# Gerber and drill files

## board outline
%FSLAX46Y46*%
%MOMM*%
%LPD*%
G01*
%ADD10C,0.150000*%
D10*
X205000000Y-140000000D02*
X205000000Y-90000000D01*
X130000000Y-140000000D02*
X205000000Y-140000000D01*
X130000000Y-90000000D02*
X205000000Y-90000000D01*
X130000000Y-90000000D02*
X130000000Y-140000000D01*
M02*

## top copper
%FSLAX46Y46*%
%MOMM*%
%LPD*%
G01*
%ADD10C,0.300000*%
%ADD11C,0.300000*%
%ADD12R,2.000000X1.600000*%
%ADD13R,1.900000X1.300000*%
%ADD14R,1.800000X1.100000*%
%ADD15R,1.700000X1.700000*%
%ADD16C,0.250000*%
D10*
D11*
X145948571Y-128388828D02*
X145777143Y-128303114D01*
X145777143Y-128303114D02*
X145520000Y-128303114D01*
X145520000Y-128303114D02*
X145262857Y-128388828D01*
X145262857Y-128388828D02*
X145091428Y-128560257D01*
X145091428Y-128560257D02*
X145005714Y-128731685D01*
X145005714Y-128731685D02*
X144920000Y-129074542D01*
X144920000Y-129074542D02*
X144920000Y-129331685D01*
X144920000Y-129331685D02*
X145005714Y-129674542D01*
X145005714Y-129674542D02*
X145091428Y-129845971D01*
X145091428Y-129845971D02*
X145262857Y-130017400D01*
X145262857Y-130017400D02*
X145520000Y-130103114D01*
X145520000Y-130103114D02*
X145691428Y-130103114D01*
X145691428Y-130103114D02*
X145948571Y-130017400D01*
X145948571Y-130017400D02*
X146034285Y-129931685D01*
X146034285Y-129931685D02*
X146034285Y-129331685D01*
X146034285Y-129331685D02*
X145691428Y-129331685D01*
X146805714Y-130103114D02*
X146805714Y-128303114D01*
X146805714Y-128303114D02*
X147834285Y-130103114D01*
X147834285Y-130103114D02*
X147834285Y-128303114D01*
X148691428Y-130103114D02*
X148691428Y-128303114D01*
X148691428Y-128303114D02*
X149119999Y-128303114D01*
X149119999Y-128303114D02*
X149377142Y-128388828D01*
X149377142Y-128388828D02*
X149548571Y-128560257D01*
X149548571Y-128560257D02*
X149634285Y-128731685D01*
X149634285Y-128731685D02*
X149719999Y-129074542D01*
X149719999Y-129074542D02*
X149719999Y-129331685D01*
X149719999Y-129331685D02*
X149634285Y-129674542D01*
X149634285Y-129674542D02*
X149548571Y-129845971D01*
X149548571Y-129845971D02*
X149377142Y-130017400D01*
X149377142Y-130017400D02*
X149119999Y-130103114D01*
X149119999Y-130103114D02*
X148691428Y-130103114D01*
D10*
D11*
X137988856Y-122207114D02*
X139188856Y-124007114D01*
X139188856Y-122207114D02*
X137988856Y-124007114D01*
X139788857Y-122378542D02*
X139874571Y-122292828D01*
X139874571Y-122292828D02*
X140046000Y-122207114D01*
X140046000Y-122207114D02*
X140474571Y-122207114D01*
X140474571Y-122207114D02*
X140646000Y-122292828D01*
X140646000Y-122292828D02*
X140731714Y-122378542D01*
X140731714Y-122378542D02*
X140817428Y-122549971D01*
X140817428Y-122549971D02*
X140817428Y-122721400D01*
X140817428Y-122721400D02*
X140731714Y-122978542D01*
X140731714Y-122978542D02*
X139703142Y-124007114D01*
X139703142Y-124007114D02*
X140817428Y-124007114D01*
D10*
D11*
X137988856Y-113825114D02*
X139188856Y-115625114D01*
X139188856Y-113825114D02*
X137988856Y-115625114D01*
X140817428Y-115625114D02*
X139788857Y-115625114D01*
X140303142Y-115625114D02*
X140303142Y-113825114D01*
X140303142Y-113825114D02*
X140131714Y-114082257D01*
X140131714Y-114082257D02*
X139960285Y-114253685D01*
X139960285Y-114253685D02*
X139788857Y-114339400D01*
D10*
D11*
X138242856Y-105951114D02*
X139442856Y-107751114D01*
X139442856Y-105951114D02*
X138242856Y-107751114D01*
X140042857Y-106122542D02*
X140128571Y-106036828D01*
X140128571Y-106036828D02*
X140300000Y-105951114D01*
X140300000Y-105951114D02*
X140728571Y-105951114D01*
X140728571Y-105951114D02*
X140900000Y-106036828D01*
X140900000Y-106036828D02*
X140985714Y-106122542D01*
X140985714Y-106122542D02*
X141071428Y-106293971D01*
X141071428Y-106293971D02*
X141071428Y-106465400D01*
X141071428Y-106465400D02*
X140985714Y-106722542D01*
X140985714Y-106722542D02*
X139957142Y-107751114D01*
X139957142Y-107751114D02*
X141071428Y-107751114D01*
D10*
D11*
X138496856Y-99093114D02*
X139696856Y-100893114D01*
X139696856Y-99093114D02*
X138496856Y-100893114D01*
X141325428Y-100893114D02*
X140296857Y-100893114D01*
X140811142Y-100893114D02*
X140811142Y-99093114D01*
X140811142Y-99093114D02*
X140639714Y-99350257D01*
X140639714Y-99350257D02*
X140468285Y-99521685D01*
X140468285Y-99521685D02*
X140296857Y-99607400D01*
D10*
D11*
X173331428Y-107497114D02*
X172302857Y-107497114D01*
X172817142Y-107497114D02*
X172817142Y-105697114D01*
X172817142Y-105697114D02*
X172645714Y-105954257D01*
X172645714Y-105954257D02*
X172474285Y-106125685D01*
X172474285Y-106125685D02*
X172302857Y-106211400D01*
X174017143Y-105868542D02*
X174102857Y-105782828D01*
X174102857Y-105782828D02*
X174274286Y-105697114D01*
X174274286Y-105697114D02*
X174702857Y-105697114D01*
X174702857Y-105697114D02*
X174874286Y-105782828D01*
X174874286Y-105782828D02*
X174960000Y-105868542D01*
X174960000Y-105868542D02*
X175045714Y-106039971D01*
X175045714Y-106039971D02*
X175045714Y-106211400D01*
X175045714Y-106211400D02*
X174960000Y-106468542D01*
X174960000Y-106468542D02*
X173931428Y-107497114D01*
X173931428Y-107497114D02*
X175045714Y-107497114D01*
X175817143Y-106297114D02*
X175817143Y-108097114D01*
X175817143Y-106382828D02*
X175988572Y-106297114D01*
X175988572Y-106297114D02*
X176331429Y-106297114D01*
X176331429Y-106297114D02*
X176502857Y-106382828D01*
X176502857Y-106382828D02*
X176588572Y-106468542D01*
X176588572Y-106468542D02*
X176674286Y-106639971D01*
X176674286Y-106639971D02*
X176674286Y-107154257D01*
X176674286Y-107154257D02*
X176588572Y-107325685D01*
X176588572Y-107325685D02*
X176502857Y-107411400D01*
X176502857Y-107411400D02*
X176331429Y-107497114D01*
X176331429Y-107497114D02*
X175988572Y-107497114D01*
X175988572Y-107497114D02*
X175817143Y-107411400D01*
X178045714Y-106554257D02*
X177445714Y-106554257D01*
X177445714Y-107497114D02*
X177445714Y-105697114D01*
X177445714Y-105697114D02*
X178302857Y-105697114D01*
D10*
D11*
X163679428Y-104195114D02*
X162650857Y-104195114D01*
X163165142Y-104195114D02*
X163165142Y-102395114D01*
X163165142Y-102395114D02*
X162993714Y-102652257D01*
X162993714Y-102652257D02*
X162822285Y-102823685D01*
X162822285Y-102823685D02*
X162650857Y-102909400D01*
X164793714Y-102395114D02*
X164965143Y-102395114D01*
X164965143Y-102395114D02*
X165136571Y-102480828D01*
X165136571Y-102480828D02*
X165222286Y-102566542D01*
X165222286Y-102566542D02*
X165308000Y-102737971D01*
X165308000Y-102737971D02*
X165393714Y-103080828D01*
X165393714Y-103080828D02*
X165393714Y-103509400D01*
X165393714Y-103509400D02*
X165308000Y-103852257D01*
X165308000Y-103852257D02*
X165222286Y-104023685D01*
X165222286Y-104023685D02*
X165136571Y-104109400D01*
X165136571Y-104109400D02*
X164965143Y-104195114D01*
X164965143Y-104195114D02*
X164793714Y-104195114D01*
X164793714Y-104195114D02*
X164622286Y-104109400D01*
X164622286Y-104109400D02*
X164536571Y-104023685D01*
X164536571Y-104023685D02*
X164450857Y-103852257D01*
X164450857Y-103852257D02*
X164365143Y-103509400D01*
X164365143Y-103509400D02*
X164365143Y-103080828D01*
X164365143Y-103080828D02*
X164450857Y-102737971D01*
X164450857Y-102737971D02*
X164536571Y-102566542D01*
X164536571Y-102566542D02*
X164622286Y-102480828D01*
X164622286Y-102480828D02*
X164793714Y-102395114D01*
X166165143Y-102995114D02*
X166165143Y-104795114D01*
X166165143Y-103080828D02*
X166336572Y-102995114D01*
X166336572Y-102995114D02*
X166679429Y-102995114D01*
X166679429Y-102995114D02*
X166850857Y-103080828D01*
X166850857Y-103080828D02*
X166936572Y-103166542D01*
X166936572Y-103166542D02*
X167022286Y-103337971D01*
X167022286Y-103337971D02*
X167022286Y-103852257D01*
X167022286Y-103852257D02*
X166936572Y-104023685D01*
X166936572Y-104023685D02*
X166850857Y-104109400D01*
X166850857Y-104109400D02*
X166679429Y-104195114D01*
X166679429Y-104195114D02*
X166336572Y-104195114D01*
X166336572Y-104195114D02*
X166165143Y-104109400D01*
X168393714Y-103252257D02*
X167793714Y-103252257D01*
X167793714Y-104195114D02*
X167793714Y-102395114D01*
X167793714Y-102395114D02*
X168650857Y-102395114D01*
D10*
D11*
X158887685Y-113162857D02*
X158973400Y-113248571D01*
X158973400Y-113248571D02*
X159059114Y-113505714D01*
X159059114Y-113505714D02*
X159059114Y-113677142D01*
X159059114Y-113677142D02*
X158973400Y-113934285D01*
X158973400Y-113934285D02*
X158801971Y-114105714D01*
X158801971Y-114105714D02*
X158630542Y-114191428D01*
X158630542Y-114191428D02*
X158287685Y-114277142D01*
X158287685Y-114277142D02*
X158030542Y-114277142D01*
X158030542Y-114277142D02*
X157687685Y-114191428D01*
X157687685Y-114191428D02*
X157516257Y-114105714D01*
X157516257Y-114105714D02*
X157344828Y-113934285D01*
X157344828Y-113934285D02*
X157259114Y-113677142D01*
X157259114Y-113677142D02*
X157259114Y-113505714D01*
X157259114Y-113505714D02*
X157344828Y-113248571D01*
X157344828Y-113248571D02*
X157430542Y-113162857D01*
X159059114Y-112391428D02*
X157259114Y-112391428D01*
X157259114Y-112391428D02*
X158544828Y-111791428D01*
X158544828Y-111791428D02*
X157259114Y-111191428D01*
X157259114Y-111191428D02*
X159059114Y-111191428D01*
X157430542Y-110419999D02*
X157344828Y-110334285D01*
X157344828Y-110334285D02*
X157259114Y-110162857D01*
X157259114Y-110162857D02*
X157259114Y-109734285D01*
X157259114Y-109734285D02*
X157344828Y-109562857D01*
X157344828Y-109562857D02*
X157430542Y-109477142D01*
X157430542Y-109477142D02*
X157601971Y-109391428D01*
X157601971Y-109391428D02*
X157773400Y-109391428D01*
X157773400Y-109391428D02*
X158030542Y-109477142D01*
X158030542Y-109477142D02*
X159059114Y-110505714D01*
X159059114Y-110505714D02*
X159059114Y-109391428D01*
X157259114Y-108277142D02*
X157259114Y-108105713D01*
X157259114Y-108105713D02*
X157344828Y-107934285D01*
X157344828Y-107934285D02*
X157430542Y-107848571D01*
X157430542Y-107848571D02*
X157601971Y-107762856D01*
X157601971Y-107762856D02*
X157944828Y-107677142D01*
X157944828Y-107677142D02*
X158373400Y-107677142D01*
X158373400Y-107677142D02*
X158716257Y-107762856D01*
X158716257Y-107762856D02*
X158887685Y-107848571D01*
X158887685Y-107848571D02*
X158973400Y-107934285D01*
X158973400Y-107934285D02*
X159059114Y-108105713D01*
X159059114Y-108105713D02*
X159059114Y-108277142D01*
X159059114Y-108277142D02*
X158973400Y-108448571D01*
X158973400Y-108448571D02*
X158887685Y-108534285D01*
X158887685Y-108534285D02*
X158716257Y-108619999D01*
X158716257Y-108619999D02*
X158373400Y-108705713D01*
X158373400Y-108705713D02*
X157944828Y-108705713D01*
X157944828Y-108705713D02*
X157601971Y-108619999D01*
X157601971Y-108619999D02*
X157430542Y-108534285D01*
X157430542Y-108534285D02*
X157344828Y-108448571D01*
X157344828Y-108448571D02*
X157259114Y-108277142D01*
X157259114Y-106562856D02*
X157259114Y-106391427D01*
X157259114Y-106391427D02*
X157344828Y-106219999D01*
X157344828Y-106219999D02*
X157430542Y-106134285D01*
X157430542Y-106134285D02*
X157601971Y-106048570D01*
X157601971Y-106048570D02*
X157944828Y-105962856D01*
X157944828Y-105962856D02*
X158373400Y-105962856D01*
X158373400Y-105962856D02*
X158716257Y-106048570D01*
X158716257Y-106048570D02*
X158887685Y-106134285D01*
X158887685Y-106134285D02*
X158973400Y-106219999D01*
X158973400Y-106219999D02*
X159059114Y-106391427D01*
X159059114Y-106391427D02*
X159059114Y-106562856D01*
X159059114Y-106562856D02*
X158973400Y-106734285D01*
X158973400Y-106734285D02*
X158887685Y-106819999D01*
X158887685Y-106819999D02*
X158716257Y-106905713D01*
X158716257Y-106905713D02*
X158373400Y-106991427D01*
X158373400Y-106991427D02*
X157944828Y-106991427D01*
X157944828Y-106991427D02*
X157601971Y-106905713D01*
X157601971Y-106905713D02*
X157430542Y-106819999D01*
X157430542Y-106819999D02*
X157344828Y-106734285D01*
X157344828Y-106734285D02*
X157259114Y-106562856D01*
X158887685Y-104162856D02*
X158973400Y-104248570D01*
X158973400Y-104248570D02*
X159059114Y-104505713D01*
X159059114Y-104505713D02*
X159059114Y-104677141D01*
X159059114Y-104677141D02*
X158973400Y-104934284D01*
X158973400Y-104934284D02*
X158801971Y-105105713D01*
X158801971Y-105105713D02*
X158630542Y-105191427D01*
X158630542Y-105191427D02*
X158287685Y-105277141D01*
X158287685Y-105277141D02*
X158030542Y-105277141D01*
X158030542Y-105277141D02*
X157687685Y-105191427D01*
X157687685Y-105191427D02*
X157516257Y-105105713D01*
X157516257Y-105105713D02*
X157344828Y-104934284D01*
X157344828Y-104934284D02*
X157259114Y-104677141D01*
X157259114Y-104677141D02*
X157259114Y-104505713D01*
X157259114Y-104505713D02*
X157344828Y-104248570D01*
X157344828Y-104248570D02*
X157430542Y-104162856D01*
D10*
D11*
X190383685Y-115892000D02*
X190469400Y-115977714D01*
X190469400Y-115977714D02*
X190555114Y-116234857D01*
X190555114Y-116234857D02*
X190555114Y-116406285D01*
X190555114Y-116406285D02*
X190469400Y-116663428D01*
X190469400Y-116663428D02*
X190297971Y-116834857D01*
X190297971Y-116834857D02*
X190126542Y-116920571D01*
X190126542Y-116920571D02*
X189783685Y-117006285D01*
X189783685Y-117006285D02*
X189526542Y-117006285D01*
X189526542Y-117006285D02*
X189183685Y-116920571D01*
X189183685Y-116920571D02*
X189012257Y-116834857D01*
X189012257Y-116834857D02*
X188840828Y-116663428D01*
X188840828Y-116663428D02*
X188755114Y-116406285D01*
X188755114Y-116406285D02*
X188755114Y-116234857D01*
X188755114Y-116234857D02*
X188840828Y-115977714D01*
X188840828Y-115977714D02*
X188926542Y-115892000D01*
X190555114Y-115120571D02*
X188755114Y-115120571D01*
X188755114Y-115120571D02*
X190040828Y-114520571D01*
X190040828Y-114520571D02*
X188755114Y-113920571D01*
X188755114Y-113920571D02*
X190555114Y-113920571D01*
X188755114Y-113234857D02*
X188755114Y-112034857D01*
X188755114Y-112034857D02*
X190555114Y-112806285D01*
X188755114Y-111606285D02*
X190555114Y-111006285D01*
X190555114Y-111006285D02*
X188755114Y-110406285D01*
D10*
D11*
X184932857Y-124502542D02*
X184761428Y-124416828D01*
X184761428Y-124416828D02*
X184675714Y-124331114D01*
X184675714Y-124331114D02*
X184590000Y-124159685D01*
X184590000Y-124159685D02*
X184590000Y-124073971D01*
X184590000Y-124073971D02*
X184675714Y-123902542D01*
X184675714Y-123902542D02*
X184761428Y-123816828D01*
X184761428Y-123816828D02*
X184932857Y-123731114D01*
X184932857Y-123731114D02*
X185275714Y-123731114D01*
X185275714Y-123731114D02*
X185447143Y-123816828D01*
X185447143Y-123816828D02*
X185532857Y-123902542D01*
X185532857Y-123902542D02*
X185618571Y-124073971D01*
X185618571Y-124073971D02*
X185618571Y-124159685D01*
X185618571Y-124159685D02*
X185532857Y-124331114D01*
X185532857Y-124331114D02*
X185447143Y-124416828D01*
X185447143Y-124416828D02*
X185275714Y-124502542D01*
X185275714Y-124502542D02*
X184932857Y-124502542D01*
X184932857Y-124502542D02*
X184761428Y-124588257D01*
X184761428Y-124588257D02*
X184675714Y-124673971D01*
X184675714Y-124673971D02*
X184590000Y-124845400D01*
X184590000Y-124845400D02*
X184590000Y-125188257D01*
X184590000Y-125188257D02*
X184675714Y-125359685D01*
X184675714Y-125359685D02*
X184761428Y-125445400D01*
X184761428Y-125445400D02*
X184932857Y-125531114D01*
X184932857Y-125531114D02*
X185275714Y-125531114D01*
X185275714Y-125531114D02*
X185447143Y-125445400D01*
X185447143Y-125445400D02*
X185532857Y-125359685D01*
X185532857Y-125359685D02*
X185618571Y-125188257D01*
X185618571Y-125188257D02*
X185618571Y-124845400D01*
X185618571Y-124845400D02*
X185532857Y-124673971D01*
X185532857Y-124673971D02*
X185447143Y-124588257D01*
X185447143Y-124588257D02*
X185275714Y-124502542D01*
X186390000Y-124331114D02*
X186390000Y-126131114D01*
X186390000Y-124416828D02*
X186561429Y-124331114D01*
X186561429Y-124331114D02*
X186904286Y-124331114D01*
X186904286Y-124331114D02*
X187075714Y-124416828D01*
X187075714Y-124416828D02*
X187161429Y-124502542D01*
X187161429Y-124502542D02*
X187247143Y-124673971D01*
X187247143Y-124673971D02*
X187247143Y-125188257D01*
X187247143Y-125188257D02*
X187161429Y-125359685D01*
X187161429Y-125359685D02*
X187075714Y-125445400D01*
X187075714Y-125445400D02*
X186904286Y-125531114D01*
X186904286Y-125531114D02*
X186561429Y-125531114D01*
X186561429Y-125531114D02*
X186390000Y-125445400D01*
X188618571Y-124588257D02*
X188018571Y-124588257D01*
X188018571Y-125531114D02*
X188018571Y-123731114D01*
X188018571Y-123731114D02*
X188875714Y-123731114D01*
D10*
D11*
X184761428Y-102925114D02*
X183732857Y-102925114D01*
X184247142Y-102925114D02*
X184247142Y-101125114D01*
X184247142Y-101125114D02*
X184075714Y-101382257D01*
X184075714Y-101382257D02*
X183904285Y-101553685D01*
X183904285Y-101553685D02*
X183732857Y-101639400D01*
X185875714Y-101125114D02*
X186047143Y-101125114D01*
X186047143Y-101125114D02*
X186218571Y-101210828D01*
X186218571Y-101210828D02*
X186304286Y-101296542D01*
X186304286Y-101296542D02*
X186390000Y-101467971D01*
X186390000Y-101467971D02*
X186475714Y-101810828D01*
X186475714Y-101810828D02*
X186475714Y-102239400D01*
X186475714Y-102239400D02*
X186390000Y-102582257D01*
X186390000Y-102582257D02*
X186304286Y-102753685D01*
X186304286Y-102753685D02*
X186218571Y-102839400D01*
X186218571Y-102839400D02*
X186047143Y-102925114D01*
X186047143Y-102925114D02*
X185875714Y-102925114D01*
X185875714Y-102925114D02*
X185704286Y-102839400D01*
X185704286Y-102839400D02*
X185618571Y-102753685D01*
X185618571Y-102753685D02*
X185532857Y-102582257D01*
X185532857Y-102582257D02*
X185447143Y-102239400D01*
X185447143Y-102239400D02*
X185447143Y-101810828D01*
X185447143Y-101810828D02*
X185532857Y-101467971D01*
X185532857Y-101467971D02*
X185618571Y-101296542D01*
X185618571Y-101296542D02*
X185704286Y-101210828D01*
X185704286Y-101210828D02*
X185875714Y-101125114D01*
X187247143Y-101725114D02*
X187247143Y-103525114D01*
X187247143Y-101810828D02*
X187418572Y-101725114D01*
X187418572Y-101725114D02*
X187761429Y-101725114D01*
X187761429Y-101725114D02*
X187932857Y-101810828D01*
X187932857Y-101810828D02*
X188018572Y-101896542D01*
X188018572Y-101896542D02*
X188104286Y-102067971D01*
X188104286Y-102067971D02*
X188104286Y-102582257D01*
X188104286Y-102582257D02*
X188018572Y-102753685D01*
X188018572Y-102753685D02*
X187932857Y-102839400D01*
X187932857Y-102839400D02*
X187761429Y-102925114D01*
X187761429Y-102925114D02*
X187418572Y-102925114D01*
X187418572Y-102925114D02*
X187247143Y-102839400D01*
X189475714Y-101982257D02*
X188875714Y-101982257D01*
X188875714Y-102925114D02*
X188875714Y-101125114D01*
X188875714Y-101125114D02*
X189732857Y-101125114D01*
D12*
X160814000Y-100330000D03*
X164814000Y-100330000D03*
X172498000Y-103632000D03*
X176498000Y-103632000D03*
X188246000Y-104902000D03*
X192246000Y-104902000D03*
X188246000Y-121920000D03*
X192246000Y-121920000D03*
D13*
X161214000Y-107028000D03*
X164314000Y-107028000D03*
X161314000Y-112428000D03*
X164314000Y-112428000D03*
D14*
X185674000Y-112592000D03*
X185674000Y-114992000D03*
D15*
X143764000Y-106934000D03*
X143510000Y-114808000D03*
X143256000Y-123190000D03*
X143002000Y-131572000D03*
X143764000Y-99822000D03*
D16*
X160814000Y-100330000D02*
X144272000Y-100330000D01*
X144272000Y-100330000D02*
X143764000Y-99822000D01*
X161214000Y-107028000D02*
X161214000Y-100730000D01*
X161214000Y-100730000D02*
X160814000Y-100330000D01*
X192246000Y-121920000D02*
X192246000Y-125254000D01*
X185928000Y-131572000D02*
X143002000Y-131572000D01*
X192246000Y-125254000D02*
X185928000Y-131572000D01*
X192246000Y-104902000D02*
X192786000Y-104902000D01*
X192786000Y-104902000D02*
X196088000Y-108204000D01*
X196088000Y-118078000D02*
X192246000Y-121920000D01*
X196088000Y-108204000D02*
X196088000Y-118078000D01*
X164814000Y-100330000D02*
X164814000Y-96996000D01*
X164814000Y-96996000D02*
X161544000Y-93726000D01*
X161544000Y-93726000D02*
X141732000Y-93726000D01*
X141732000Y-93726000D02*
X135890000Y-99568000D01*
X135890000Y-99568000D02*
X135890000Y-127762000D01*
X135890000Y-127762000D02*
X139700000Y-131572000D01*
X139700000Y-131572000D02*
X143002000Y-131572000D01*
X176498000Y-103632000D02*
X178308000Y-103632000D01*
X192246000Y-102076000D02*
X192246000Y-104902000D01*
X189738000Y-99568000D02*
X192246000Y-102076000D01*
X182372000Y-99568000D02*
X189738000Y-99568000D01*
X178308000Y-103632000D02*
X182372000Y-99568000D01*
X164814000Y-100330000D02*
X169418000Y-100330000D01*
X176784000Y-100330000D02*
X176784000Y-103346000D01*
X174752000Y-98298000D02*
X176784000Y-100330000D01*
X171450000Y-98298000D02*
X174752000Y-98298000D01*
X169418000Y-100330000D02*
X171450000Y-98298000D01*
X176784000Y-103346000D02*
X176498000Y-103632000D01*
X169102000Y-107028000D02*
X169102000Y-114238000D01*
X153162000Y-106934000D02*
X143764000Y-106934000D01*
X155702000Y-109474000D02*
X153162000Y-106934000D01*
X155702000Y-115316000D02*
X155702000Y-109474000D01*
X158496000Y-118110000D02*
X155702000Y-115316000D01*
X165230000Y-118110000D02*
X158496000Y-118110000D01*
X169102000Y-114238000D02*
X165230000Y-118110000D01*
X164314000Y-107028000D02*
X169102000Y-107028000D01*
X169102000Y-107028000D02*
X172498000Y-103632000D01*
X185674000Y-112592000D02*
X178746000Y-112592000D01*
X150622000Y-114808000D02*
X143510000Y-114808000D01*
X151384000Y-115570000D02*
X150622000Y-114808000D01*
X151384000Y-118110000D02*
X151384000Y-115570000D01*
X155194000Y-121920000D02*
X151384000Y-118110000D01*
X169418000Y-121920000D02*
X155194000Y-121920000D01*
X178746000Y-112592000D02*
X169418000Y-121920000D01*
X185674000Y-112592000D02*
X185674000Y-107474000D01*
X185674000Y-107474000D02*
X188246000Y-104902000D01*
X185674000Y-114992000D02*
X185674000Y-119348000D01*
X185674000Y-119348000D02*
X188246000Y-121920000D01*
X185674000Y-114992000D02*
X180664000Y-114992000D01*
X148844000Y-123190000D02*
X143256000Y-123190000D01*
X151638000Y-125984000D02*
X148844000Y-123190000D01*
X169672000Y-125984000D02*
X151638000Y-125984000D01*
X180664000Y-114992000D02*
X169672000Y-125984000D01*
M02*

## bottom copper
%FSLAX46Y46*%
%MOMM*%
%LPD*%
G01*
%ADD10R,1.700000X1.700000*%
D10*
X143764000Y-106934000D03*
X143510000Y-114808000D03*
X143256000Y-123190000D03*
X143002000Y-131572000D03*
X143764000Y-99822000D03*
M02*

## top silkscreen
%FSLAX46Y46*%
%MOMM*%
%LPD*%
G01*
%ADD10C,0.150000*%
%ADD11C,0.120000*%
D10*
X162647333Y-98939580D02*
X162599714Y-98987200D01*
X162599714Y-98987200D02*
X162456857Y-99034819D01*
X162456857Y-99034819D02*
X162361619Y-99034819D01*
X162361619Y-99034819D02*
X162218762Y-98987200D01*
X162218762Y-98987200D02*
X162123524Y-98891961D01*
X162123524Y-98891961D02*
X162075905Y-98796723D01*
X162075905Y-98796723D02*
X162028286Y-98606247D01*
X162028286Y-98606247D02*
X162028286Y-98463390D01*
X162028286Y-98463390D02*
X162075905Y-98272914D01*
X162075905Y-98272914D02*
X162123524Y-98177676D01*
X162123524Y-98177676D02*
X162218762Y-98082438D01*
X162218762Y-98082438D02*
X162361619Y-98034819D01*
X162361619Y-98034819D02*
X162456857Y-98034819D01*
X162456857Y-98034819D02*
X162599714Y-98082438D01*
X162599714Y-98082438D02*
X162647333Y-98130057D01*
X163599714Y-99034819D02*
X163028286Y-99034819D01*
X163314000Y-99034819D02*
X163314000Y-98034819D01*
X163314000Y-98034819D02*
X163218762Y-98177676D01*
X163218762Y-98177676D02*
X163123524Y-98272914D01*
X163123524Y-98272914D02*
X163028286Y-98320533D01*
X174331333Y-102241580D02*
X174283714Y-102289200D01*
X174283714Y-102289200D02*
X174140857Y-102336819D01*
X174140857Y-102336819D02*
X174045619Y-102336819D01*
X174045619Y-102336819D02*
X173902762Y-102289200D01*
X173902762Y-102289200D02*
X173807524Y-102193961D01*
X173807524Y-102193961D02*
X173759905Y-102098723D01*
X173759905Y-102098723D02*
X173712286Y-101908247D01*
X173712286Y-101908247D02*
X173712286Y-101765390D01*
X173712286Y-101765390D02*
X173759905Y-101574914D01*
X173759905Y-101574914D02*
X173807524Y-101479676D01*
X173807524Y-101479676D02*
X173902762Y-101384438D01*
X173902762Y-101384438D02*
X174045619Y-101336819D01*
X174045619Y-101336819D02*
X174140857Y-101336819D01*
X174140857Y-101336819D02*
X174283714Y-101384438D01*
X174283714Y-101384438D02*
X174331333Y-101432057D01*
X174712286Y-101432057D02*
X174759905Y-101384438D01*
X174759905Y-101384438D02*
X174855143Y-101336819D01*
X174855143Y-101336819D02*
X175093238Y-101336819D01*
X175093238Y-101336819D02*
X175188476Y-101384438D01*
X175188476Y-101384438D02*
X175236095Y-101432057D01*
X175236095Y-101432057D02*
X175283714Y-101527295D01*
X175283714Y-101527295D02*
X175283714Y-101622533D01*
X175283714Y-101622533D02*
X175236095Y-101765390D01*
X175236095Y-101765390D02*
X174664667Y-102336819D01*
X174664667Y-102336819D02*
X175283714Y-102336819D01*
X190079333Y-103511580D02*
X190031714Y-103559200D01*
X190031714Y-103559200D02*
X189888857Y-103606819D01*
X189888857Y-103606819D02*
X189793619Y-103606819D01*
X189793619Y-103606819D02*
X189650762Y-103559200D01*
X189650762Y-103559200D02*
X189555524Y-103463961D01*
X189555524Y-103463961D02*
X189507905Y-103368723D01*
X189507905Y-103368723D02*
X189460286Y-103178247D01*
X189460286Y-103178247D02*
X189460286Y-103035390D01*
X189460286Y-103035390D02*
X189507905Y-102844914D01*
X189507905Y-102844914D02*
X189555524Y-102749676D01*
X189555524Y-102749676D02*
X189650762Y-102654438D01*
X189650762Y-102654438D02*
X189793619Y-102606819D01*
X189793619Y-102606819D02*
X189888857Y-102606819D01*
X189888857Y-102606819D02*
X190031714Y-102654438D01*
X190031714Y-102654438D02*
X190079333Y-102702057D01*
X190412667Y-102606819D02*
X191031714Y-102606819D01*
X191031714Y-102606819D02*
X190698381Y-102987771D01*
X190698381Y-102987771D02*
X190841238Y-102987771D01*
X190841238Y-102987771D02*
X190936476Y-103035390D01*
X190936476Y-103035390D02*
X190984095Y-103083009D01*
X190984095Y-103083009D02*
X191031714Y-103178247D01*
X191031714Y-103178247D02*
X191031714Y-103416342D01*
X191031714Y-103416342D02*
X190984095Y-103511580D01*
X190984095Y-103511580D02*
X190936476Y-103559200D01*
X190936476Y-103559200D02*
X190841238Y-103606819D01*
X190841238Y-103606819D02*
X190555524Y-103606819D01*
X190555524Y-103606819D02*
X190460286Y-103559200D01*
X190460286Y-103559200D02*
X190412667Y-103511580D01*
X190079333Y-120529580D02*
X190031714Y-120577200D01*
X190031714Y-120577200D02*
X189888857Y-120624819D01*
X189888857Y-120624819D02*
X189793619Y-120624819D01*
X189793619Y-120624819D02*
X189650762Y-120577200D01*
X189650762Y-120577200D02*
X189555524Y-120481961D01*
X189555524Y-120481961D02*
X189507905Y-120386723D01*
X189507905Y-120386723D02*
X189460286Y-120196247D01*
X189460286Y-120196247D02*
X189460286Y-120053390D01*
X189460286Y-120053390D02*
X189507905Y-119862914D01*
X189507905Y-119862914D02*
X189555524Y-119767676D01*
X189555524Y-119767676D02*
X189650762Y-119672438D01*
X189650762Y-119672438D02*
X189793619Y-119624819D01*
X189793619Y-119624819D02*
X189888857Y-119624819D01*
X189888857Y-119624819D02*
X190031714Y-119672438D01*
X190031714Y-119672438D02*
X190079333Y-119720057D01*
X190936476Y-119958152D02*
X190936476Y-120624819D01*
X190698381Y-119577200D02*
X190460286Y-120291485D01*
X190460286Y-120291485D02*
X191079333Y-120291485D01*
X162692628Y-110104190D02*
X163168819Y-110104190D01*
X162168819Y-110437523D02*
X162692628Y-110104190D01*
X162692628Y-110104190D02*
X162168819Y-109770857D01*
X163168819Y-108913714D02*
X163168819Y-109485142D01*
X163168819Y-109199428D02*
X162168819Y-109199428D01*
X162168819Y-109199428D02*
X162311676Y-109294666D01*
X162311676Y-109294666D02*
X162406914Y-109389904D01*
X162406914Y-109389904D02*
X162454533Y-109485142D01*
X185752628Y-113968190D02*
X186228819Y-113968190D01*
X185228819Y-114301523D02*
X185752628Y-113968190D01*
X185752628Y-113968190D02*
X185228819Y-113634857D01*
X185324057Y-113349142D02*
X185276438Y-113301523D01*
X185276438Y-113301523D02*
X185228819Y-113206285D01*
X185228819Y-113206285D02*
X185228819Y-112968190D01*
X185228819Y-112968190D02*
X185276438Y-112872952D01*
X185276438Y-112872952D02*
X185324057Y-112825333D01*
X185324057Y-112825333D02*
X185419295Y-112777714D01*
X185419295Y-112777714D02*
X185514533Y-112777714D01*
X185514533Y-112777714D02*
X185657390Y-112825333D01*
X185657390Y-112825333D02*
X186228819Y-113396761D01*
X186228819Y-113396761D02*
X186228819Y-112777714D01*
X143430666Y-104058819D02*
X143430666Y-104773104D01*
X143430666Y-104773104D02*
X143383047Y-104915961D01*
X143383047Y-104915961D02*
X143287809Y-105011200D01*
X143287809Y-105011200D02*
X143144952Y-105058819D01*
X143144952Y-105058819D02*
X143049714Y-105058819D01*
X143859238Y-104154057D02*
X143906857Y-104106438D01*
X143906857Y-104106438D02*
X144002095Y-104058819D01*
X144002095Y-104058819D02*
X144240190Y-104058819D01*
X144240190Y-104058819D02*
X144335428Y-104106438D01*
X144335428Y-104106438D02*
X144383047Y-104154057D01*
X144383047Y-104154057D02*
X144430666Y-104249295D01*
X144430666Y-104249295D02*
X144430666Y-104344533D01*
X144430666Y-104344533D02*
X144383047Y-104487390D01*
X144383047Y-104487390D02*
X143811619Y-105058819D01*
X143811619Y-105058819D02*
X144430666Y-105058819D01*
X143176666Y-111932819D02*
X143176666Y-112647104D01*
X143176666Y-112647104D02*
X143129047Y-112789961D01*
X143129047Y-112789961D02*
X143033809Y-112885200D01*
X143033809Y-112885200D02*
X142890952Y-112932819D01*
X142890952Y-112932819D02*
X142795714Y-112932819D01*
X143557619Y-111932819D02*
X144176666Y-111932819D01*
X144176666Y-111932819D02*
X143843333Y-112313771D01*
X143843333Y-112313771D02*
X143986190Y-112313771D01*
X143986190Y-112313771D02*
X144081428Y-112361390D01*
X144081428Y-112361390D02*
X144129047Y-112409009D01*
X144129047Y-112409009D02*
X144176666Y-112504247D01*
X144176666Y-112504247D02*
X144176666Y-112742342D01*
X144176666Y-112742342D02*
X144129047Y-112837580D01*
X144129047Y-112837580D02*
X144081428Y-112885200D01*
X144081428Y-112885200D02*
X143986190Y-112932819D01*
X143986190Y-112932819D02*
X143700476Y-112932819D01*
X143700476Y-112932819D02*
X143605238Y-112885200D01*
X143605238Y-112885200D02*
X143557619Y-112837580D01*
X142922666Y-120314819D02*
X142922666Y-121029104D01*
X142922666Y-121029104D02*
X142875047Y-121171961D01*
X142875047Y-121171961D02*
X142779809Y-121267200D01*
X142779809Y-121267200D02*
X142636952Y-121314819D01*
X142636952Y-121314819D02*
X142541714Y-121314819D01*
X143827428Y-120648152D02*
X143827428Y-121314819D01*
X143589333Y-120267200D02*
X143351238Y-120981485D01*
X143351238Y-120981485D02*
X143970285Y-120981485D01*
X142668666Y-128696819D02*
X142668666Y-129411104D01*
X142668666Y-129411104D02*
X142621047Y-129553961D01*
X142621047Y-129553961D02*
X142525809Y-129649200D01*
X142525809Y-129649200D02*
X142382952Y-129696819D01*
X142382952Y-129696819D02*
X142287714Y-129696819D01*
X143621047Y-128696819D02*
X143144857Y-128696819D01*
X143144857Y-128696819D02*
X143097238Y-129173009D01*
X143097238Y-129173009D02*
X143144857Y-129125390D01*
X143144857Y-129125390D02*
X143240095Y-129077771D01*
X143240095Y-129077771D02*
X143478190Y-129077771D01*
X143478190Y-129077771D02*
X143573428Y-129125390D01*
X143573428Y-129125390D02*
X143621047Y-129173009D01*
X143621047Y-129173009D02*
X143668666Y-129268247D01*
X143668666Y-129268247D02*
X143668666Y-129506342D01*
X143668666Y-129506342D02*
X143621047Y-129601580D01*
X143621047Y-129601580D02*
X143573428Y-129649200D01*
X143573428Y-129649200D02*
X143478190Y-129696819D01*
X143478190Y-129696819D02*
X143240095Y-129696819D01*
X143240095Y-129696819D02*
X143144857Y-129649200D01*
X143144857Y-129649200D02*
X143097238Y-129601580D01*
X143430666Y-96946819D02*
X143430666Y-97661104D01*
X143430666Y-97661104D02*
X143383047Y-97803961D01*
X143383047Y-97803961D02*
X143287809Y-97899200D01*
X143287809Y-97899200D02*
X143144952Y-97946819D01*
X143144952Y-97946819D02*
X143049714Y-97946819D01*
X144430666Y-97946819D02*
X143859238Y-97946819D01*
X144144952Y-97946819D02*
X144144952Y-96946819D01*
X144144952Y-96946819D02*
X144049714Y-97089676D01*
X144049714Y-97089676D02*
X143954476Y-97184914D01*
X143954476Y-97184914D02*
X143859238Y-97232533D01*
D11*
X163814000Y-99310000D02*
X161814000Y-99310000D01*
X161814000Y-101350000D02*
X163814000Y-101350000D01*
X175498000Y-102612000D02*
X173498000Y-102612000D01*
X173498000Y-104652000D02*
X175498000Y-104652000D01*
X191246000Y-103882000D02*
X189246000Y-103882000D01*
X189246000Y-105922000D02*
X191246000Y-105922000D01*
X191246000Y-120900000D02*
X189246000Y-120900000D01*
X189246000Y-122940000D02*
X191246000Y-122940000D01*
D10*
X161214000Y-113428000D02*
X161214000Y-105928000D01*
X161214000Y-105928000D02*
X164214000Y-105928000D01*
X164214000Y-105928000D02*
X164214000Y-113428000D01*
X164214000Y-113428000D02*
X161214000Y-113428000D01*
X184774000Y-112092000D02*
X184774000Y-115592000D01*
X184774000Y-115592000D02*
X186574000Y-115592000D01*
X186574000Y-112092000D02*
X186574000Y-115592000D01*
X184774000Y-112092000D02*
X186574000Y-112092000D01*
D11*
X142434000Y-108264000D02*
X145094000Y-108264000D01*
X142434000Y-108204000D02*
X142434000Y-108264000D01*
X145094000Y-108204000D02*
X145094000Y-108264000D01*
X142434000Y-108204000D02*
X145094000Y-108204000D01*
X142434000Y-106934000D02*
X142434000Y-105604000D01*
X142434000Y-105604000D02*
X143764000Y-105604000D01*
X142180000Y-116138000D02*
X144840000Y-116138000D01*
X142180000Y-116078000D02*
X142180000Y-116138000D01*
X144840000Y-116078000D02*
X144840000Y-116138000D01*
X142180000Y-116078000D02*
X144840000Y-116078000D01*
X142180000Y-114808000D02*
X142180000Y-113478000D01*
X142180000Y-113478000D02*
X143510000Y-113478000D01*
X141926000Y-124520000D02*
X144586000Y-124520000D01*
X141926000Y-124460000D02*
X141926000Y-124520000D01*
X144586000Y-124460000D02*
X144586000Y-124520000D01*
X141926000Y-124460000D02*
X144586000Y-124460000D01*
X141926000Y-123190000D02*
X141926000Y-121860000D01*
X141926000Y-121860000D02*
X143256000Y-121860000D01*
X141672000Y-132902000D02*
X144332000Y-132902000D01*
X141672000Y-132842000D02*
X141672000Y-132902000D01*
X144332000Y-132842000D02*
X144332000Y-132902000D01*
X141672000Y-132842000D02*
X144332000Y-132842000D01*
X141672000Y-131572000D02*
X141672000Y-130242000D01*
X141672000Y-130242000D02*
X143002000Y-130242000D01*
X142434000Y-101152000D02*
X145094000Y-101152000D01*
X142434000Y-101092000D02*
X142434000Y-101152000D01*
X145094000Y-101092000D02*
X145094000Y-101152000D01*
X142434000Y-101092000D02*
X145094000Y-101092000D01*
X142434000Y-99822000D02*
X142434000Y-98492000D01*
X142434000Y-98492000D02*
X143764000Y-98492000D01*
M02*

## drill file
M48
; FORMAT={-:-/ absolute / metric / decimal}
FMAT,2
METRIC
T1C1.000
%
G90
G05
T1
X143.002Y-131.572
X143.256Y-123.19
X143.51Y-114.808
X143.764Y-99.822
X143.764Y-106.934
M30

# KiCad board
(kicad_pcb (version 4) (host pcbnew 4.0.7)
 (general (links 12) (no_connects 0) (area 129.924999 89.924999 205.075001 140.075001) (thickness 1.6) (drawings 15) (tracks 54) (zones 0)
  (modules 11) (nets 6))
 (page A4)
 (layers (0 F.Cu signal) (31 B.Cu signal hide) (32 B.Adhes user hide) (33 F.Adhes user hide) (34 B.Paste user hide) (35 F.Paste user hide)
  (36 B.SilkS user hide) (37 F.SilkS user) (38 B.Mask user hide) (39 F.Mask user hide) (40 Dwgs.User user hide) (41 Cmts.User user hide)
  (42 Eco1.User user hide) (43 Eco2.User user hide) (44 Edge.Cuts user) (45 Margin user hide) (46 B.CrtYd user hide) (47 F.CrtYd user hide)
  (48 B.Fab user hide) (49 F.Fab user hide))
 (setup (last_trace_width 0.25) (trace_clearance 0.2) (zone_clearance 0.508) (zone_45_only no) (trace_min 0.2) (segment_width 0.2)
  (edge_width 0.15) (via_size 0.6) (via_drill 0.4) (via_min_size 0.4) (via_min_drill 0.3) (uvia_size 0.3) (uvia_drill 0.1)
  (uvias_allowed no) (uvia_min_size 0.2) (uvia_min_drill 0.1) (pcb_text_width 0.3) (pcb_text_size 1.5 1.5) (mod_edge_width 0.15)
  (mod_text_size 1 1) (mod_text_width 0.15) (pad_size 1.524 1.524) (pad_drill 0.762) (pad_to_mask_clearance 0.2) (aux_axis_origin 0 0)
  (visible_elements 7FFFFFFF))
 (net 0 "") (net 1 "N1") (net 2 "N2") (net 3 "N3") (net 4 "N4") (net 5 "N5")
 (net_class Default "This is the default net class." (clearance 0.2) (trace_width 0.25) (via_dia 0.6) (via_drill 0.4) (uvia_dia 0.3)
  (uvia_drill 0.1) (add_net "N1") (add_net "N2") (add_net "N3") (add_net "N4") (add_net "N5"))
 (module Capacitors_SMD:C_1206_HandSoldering (layer F.Cu) (at 162.814 100.33)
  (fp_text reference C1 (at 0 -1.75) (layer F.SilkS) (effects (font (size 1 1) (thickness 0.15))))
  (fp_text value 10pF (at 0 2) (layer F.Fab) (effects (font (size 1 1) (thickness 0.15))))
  (fp_line (start 1 -1.02) (end -1 -1.02) (layer F.SilkS) (width 0.12))
  (fp_line (start -1 1.02) (end 1 1.02) (layer F.SilkS) (width 0.12))
  (pad 1 smd rect (at -2 0) (size 2 1.6) (layers F.Cu F.Paste F.Mask) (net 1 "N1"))
  (pad 2 smd rect (at 2 0) (size 2 1.6) (layers F.Cu F.Paste F.Mask) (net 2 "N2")))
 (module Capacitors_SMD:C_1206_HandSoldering (layer F.Cu) (at 174.498 103.632)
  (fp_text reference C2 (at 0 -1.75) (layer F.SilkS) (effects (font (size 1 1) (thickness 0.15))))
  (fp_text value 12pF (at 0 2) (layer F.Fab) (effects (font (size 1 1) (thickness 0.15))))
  (fp_line (start 1 -1.02) (end -1 -1.02) (layer F.SilkS) (width 0.12))
  (fp_line (start -1 1.02) (end 1 1.02) (layer F.SilkS) (width 0.12))
  (pad 1 smd rect (at -2 0) (size 2 1.6) (layers F.Cu F.Paste F.Mask) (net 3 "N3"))
  (pad 2 smd rect (at 2 0) (size 2 1.6) (layers F.Cu F.Paste F.Mask) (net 2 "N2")))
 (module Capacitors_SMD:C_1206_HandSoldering (layer F.Cu) (at 190.246 104.902)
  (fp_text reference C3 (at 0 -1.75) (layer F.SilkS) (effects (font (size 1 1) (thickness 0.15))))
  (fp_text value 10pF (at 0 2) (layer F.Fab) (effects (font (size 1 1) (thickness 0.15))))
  (fp_line (start 1 -1.02) (end -1 -1.02) (layer F.SilkS) (width 0.12))
  (fp_line (start -1 1.02) (end 1 1.02) (layer F.SilkS) (width 0.12))
  (pad 1 smd rect (at -2 0) (size 2 1.6) (layers F.Cu F.Paste F.Mask) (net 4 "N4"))
  (pad 2 smd rect (at 2 0) (size 2 1.6) (layers F.Cu F.Paste F.Mask) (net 2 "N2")))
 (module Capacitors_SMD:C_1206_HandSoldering (layer F.Cu) (at 190.246 121.92)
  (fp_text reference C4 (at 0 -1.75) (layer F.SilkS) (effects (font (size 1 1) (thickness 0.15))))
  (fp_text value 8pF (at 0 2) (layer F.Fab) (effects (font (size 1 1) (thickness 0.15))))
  (fp_line (start 1 -1.02) (end -1 -1.02) (layer F.SilkS) (width 0.12))
  (fp_line (start -1 1.02) (end 1 1.02) (layer F.SilkS) (width 0.12))
  (pad 1 smd rect (at -2 0) (size 2 1.6) (layers F.Cu F.Paste F.Mask) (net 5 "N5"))
  (pad 2 smd rect (at 2 0) (size 2 1.6) (layers F.Cu F.Paste F.Mask) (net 2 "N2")))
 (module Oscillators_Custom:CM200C (layer F.Cu) (at 162.814 109.728 90)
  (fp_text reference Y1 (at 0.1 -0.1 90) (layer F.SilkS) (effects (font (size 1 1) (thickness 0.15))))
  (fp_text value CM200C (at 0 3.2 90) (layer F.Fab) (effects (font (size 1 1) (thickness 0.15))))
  (fp_line (start -3.7 -1.6) (end 3.8 -1.6) (layer F.SilkS) (width 0.15))
  (fp_line (start 3.8 -1.6) (end 3.8 1.4) (layer F.SilkS) (width 0.15))
  (fp_line (start 3.8 1.4) (end -3.7 1.4) (layer F.SilkS) (width 0.15))
  (fp_line (start -3.7 1.4) (end -3.7 -1.6) (layer F.SilkS) (width 0.15))
  (pad 1 smd rect (at 2.7 -1.6 90) (size 1.3 1.9) (layers F.Cu F.Paste F.Mask) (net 1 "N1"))
  (pad 2 smd rect (at 2.7 1.5 90) (size 1.3 1.9) (layers F.Cu F.Paste F.Mask) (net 3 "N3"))
  (pad 3 smd rect (at -2.7 -1.5 90) (size 1.3 1.9) (layers F.Cu F.Paste F.Mask))
  (pad 4 smd rect (at -2.7 1.5 90) (size 1.3 1.9) (layers F.Cu F.Paste F.Mask)))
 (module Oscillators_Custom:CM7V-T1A (layer F.Cu) (at 185.674 113.792 90)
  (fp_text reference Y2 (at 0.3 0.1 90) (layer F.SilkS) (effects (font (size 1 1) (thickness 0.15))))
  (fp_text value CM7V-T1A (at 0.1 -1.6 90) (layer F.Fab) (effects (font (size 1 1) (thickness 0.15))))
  (fp_line (start 1.7 -0.9) (end -1.8 -0.9) (layer F.SilkS) (width 0.15))
  (fp_line (start -1.8 -0.9) (end -1.8 0.9) (layer F.SilkS) (width 0.15))
  (fp_line (start 1.7 0.9) (end -1.8 0.9) (layer F.SilkS) (width 0.15))
  (fp_line (start 1.7 -0.9) (end 1.7 0.9) (layer F.SilkS) (width 0.15))
  (pad 1 smd rect (at 1.2 0 90) (size 1.1 1.8) (layers F.Cu F.Paste F.Mask) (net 4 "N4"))
  (pad 2 smd rect (at -1.2 0 90) (size 1.1 1.8) (layers F.Cu F.Paste F.Mask) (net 5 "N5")))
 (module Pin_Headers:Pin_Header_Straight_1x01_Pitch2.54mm (layer F.Cu) (at 143.764 106.934)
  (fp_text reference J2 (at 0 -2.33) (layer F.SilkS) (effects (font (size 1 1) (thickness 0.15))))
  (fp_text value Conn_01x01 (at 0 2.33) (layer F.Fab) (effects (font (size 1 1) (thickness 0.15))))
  (fp_line (start -1.33 1.33) (end 1.33 1.33) (layer F.SilkS) (width 0.12))
  (fp_line (start -1.33 1.27) (end -1.33 1.33) (layer F.SilkS) (width 0.12))
  (fp_line (start 1.33 1.27) (end 1.33 1.33) (layer F.SilkS) (width 0.12))
  (fp_line (start -1.33 1.27) (end 1.33 1.27) (layer F.SilkS) (width 0.12))
  (fp_line (start -1.33 0) (end -1.33 -1.33) (layer F.SilkS) (width 0.12))
  (fp_line (start -1.33 -1.33) (end 0 -1.33) (layer F.SilkS) (width 0.12))
  (pad 1 thru_hole rect (at 0 0) (size 1.7 1.7) (drill 1) (layers *.Cu *.Mask) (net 3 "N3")))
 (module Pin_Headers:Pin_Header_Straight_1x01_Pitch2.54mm (layer F.Cu) (at 143.51 114.808)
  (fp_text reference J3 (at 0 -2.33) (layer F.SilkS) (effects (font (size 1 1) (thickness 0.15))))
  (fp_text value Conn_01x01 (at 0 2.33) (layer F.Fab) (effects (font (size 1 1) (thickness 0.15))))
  (fp_line (start -1.33 1.33) (end 1.33 1.33) (layer F.SilkS) (width 0.12))
  (fp_line (start -1.33 1.27) (end -1.33 1.33) (layer F.SilkS) (width 0.12))
  (fp_line (start 1.33 1.27) (end 1.33 1.33) (layer F.SilkS) (width 0.12))
  (fp_line (start -1.33 1.27) (end 1.33 1.27) (layer F.SilkS) (width 0.12))
  (fp_line (start -1.33 0) (end -1.33 -1.33) (layer F.SilkS) (width 0.12))
  (fp_line (start -1.33 -1.33) (end 0 -1.33) (layer F.SilkS) (width 0.12))
  (pad 1 thru_hole rect (at 0 0) (size 1.7 1.7) (drill 1) (layers *.Cu *.Mask) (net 4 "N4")))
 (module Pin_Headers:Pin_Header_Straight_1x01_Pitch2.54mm (layer F.Cu) (at 143.256 123.19)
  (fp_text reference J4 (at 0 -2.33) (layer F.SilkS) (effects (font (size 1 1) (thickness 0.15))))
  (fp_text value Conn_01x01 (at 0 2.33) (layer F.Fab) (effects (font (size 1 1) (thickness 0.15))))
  (fp_line (start -1.33 1.33) (end 1.33 1.33) (layer F.SilkS) (width 0.12))
  (fp_line (start -1.33 1.27) (end -1.33 1.33) (layer F.SilkS) (width 0.12))
  (fp_line (start 1.33 1.27) (end 1.33 1.33) (layer F.SilkS) (width 0.12))
  (fp_line (start -1.33 1.27) (end 1.33 1.27) (layer F.SilkS) (width 0.12))
  (fp_line (start -1.33 0) (end -1.33 -1.33) (layer F.SilkS) (width 0.12))
  (fp_line (start -1.33 -1.33) (end 0 -1.33) (layer F.SilkS) (width 0.12))
  (pad 1 thru_hole rect (at 0 0) (size 1.7 1.7) (drill 1) (layers *.Cu *.Mask) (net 5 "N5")))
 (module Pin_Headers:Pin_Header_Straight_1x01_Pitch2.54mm (layer F.Cu) (at 143.002 131.572)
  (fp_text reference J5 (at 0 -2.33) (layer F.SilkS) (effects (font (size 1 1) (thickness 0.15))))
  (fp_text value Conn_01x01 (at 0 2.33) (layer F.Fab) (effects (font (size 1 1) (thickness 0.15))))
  (fp_line (start -1.33 1.33) (end 1.33 1.33) (layer F.SilkS) (width 0.12))
  (fp_line (start -1.33 1.27) (end -1.33 1.33) (layer F.SilkS) (width 0.12))
  (fp_line (start 1.33 1.27) (end 1.33 1.33) (layer F.SilkS) (width 0.12))
  (fp_line (start -1.33 1.27) (end 1.33 1.27) (layer F.SilkS) (width 0.12))
  (fp_line (start -1.33 0) (end -1.33 -1.33) (layer F.SilkS) (width 0.12))
  (fp_line (start -1.33 -1.33) (end 0 -1.33) (layer F.SilkS) (width 0.12))
  (pad 1 thru_hole rect (at 0 0) (size 1.7 1.7) (drill 1) (layers *.Cu *.Mask) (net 2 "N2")))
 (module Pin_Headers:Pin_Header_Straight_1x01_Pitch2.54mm (layer F.Cu) (at 143.764 99.822)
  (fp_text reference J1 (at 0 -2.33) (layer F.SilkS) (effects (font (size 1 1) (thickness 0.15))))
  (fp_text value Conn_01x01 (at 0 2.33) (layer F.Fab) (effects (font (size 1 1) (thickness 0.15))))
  (fp_line (start -1.33 1.33) (end 1.33 1.33) (layer F.SilkS) (width 0.12))
  (fp_line (start -1.33 1.27) (end -1.33 1.33) (layer F.SilkS) (width 0.12))
  (fp_line (start 1.33 1.27) (end 1.33 1.33) (layer F.SilkS) (width 0.12))
  (fp_line (start -1.33 1.27) (end 1.33 1.27) (layer F.SilkS) (width 0.12))
  (fp_line (start -1.33 0) (end -1.33 -1.33) (layer F.SilkS) (width 0.12))
  (fp_line (start -1.33 -1.33) (end 0 -1.33) (layer F.SilkS) (width 0.12))
  (pad 1 thru_hole rect (at 0 0) (size 1.7 1.7) (drill 1) (layers *.Cu *.Mask) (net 1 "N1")))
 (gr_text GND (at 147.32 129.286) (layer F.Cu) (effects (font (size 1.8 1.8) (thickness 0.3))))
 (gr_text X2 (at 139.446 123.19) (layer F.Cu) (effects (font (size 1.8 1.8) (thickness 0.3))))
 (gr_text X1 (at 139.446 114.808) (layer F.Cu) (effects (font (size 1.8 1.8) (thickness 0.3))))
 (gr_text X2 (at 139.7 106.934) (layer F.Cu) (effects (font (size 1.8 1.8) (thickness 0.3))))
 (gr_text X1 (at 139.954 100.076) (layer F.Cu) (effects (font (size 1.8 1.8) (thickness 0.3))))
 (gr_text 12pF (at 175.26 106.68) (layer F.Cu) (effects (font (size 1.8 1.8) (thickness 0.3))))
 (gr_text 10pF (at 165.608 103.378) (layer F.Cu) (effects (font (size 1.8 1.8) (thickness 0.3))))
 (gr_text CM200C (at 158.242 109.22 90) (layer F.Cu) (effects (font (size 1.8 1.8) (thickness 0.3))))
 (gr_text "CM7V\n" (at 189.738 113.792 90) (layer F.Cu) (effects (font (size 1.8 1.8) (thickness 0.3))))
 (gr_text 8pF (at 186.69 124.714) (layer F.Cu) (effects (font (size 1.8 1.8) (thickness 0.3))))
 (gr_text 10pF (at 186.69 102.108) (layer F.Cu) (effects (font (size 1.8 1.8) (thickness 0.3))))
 (gr_line (start 205 140) (end 205 90) (angle 90) (layer Edge.Cuts) (width 0.15))
 (gr_line (start 130 140) (end 205 140) (angle 90) (layer Edge.Cuts) (width 0.15))
 (gr_line (start 130 90) (end 205 90) (angle 90) (layer Edge.Cuts) (width 0.15))
 (gr_line (start 130 90) (end 130 140) (angle 90) (layer Edge.Cuts) (width 0.15))
 (segment (start 160.814 100.33) (end 144.272 100.33) (width 0.25) (layer F.Cu) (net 1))
 (segment (start 144.272 100.33) (end 143.764 99.822) (width 0.25) (layer F.Cu) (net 1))
 (segment (start 161.214 107.028) (end 161.214 100.73) (width 0.25) (layer F.Cu) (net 1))
 (segment (start 161.214 100.73) (end 160.814 100.33) (width 0.25) (layer F.Cu) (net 1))
 (segment (start 192.246 121.92) (end 192.246 125.254) (width 0.25) (layer F.Cu) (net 2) (status 400000))
 (segment (start 185.928 131.572) (end 143.002 131.572) (width 0.25) (layer F.Cu) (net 2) (status 800000))
 (segment (start 192.246 125.254) (end 185.928 131.572) (width 0.25) (layer F.Cu) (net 2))
 (segment (start 192.246 104.902) (end 192.786 104.902) (width 0.25) (layer F.Cu) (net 2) (status C00000))
 (segment (start 192.786 104.902) (end 196.088 108.204) (width 0.25) (layer F.Cu) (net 2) (status 400000))
 (segment (start 196.088 118.078) (end 192.246 121.92) (width 0.25) (layer F.Cu) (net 2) (status 800000))
 (segment (start 196.088 108.204) (end 196.088 118.078) (width 0.25) (layer F.Cu) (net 2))
 (segment (start 164.814 100.33) (end 164.814 96.996) (width 0.25) (layer F.Cu) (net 2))
 (segment (start 164.814 96.996) (end 161.544 93.726) (width 0.25) (layer F.Cu) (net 2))
 (segment (start 161.544 93.726) (end 141.732 93.726) (width 0.25) (layer F.Cu) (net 2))
 (segment (start 141.732 93.726) (end 135.89 99.568) (width 0.25) (layer F.Cu) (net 2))
 (segment (start 135.89 99.568) (end 135.89 127.762) (width 0.25) (layer F.Cu) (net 2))
 (segment (start 135.89 127.762) (end 139.7 131.572) (width 0.25) (layer F.Cu) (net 2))
 (segment (start 139.7 131.572) (end 143.002 131.572) (width 0.25) (layer F.Cu) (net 2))
 (segment (start 176.498 103.632) (end 178.308 103.632) (width 0.25) (layer F.Cu) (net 2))
 (segment (start 192.246 102.076) (end 192.246 104.902) (width 0.25) (layer F.Cu) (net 2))
 (segment (start 189.738 99.568) (end 192.246 102.076) (width 0.25) (layer F.Cu) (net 2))
 (segment (start 182.372 99.568) (end 189.738 99.568) (width 0.25) (layer F.Cu) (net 2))
 (segment (start 178.308 103.632) (end 182.372 99.568) (width 0.25) (layer F.Cu) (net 2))
 (segment (start 164.814 100.33) (end 169.418 100.33) (width 0.25) (layer F.Cu) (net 2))
 (segment (start 176.784 100.33) (end 176.784 103.346) (width 0.25) (layer F.Cu) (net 2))
 (segment (start 174.752 98.298) (end 176.784 100.33) (width 0.25) (layer F.Cu) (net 2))
 (segment (start 171.45 98.298) (end 174.752 98.298) (width 0.25) (layer F.Cu) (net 2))
 (segment (start 169.418 100.33) (end 171.45 98.298) (width 0.25) (layer F.Cu) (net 2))
 (segment (start 176.784 103.346) (end 176.498 103.632) (width 0.25) (layer F.Cu) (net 2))
 (segment (start 169.102 107.028) (end 169.102 114.238) (width 0.25) (layer F.Cu) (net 3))
 (segment (start 153.162 106.934) (end 143.764 106.934) (width 0.25) (layer F.Cu) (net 3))
 (segment (start 155.702 109.474) (end 153.162 106.934) (width 0.25) (layer F.Cu) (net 3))
 (segment (start 155.702 115.316) (end 155.702 109.474) (width 0.25) (layer F.Cu) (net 3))
 (segment (start 158.496 118.11) (end 155.702 115.316) (width 0.25) (layer F.Cu) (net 3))
 (segment (start 165.23 118.11) (end 158.496 118.11) (width 0.25) (layer F.Cu) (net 3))
 (segment (start 169.102 114.238) (end 165.23 118.11) (width 0.25) (layer F.Cu) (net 3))
 (segment (start 164.314 107.028) (end 169.102 107.028) (width 0.25) (layer F.Cu) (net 3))
 (segment (start 169.102 107.028) (end 172.498 103.632) (width 0.25) (layer F.Cu) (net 3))
 (segment (start 185.674 112.592) (end 178.746 112.592) (width 0.25) (layer F.Cu) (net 4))
 (segment (start 150.622 114.808) (end 143.51 114.808) (width 0.25) (layer F.Cu) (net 4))
 (segment (start 151.384 115.57) (end 150.622 114.808) (width 0.25) (layer F.Cu) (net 4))
 (segment (start 151.384 118.11) (end 151.384 115.57) (width 0.25) (layer F.Cu) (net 4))
 (segment (start 155.194 121.92) (end 151.384 118.11) (width 0.25) (layer F.Cu) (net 4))
 (segment (start 169.418 121.92) (end 155.194 121.92) (width 0.25) (layer F.Cu) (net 4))
 (segment (start 178.746 112.592) (end 169.418 121.92) (width 0.25) (layer F.Cu) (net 4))
 (segment (start 185.674 112.592) (end 185.674 107.474) (width 0.25) (layer F.Cu) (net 4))
 (segment (start 185.674 107.474) (end 188.246 104.902) (width 0.25) (layer F.Cu) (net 4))
 (segment (start 185.674 114.992) (end 185.674 119.348) (width 0.25) (layer F.Cu) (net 5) (status 400000))
 (segment (start 185.674 119.348) (end 188.246 121.92) (width 0.25) (layer F.Cu) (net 5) (status 800000))
 (segment (start 185.674 114.992) (end 180.664 114.992) (width 0.25) (layer F.Cu) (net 5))
 (segment (start 148.844 123.19) (end 143.256 123.19) (width 0.25) (layer F.Cu) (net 5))
 (segment (start 151.638 125.984) (end 148.844 123.19) (width 0.25) (layer F.Cu) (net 5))
 (segment (start 169.672 125.984) (end 151.638 125.984) (width 0.25) (layer F.Cu) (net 5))
 (segment (start 180.664 114.992) (end 169.672 125.984) (width 0.25) (layer F.Cu) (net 5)))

